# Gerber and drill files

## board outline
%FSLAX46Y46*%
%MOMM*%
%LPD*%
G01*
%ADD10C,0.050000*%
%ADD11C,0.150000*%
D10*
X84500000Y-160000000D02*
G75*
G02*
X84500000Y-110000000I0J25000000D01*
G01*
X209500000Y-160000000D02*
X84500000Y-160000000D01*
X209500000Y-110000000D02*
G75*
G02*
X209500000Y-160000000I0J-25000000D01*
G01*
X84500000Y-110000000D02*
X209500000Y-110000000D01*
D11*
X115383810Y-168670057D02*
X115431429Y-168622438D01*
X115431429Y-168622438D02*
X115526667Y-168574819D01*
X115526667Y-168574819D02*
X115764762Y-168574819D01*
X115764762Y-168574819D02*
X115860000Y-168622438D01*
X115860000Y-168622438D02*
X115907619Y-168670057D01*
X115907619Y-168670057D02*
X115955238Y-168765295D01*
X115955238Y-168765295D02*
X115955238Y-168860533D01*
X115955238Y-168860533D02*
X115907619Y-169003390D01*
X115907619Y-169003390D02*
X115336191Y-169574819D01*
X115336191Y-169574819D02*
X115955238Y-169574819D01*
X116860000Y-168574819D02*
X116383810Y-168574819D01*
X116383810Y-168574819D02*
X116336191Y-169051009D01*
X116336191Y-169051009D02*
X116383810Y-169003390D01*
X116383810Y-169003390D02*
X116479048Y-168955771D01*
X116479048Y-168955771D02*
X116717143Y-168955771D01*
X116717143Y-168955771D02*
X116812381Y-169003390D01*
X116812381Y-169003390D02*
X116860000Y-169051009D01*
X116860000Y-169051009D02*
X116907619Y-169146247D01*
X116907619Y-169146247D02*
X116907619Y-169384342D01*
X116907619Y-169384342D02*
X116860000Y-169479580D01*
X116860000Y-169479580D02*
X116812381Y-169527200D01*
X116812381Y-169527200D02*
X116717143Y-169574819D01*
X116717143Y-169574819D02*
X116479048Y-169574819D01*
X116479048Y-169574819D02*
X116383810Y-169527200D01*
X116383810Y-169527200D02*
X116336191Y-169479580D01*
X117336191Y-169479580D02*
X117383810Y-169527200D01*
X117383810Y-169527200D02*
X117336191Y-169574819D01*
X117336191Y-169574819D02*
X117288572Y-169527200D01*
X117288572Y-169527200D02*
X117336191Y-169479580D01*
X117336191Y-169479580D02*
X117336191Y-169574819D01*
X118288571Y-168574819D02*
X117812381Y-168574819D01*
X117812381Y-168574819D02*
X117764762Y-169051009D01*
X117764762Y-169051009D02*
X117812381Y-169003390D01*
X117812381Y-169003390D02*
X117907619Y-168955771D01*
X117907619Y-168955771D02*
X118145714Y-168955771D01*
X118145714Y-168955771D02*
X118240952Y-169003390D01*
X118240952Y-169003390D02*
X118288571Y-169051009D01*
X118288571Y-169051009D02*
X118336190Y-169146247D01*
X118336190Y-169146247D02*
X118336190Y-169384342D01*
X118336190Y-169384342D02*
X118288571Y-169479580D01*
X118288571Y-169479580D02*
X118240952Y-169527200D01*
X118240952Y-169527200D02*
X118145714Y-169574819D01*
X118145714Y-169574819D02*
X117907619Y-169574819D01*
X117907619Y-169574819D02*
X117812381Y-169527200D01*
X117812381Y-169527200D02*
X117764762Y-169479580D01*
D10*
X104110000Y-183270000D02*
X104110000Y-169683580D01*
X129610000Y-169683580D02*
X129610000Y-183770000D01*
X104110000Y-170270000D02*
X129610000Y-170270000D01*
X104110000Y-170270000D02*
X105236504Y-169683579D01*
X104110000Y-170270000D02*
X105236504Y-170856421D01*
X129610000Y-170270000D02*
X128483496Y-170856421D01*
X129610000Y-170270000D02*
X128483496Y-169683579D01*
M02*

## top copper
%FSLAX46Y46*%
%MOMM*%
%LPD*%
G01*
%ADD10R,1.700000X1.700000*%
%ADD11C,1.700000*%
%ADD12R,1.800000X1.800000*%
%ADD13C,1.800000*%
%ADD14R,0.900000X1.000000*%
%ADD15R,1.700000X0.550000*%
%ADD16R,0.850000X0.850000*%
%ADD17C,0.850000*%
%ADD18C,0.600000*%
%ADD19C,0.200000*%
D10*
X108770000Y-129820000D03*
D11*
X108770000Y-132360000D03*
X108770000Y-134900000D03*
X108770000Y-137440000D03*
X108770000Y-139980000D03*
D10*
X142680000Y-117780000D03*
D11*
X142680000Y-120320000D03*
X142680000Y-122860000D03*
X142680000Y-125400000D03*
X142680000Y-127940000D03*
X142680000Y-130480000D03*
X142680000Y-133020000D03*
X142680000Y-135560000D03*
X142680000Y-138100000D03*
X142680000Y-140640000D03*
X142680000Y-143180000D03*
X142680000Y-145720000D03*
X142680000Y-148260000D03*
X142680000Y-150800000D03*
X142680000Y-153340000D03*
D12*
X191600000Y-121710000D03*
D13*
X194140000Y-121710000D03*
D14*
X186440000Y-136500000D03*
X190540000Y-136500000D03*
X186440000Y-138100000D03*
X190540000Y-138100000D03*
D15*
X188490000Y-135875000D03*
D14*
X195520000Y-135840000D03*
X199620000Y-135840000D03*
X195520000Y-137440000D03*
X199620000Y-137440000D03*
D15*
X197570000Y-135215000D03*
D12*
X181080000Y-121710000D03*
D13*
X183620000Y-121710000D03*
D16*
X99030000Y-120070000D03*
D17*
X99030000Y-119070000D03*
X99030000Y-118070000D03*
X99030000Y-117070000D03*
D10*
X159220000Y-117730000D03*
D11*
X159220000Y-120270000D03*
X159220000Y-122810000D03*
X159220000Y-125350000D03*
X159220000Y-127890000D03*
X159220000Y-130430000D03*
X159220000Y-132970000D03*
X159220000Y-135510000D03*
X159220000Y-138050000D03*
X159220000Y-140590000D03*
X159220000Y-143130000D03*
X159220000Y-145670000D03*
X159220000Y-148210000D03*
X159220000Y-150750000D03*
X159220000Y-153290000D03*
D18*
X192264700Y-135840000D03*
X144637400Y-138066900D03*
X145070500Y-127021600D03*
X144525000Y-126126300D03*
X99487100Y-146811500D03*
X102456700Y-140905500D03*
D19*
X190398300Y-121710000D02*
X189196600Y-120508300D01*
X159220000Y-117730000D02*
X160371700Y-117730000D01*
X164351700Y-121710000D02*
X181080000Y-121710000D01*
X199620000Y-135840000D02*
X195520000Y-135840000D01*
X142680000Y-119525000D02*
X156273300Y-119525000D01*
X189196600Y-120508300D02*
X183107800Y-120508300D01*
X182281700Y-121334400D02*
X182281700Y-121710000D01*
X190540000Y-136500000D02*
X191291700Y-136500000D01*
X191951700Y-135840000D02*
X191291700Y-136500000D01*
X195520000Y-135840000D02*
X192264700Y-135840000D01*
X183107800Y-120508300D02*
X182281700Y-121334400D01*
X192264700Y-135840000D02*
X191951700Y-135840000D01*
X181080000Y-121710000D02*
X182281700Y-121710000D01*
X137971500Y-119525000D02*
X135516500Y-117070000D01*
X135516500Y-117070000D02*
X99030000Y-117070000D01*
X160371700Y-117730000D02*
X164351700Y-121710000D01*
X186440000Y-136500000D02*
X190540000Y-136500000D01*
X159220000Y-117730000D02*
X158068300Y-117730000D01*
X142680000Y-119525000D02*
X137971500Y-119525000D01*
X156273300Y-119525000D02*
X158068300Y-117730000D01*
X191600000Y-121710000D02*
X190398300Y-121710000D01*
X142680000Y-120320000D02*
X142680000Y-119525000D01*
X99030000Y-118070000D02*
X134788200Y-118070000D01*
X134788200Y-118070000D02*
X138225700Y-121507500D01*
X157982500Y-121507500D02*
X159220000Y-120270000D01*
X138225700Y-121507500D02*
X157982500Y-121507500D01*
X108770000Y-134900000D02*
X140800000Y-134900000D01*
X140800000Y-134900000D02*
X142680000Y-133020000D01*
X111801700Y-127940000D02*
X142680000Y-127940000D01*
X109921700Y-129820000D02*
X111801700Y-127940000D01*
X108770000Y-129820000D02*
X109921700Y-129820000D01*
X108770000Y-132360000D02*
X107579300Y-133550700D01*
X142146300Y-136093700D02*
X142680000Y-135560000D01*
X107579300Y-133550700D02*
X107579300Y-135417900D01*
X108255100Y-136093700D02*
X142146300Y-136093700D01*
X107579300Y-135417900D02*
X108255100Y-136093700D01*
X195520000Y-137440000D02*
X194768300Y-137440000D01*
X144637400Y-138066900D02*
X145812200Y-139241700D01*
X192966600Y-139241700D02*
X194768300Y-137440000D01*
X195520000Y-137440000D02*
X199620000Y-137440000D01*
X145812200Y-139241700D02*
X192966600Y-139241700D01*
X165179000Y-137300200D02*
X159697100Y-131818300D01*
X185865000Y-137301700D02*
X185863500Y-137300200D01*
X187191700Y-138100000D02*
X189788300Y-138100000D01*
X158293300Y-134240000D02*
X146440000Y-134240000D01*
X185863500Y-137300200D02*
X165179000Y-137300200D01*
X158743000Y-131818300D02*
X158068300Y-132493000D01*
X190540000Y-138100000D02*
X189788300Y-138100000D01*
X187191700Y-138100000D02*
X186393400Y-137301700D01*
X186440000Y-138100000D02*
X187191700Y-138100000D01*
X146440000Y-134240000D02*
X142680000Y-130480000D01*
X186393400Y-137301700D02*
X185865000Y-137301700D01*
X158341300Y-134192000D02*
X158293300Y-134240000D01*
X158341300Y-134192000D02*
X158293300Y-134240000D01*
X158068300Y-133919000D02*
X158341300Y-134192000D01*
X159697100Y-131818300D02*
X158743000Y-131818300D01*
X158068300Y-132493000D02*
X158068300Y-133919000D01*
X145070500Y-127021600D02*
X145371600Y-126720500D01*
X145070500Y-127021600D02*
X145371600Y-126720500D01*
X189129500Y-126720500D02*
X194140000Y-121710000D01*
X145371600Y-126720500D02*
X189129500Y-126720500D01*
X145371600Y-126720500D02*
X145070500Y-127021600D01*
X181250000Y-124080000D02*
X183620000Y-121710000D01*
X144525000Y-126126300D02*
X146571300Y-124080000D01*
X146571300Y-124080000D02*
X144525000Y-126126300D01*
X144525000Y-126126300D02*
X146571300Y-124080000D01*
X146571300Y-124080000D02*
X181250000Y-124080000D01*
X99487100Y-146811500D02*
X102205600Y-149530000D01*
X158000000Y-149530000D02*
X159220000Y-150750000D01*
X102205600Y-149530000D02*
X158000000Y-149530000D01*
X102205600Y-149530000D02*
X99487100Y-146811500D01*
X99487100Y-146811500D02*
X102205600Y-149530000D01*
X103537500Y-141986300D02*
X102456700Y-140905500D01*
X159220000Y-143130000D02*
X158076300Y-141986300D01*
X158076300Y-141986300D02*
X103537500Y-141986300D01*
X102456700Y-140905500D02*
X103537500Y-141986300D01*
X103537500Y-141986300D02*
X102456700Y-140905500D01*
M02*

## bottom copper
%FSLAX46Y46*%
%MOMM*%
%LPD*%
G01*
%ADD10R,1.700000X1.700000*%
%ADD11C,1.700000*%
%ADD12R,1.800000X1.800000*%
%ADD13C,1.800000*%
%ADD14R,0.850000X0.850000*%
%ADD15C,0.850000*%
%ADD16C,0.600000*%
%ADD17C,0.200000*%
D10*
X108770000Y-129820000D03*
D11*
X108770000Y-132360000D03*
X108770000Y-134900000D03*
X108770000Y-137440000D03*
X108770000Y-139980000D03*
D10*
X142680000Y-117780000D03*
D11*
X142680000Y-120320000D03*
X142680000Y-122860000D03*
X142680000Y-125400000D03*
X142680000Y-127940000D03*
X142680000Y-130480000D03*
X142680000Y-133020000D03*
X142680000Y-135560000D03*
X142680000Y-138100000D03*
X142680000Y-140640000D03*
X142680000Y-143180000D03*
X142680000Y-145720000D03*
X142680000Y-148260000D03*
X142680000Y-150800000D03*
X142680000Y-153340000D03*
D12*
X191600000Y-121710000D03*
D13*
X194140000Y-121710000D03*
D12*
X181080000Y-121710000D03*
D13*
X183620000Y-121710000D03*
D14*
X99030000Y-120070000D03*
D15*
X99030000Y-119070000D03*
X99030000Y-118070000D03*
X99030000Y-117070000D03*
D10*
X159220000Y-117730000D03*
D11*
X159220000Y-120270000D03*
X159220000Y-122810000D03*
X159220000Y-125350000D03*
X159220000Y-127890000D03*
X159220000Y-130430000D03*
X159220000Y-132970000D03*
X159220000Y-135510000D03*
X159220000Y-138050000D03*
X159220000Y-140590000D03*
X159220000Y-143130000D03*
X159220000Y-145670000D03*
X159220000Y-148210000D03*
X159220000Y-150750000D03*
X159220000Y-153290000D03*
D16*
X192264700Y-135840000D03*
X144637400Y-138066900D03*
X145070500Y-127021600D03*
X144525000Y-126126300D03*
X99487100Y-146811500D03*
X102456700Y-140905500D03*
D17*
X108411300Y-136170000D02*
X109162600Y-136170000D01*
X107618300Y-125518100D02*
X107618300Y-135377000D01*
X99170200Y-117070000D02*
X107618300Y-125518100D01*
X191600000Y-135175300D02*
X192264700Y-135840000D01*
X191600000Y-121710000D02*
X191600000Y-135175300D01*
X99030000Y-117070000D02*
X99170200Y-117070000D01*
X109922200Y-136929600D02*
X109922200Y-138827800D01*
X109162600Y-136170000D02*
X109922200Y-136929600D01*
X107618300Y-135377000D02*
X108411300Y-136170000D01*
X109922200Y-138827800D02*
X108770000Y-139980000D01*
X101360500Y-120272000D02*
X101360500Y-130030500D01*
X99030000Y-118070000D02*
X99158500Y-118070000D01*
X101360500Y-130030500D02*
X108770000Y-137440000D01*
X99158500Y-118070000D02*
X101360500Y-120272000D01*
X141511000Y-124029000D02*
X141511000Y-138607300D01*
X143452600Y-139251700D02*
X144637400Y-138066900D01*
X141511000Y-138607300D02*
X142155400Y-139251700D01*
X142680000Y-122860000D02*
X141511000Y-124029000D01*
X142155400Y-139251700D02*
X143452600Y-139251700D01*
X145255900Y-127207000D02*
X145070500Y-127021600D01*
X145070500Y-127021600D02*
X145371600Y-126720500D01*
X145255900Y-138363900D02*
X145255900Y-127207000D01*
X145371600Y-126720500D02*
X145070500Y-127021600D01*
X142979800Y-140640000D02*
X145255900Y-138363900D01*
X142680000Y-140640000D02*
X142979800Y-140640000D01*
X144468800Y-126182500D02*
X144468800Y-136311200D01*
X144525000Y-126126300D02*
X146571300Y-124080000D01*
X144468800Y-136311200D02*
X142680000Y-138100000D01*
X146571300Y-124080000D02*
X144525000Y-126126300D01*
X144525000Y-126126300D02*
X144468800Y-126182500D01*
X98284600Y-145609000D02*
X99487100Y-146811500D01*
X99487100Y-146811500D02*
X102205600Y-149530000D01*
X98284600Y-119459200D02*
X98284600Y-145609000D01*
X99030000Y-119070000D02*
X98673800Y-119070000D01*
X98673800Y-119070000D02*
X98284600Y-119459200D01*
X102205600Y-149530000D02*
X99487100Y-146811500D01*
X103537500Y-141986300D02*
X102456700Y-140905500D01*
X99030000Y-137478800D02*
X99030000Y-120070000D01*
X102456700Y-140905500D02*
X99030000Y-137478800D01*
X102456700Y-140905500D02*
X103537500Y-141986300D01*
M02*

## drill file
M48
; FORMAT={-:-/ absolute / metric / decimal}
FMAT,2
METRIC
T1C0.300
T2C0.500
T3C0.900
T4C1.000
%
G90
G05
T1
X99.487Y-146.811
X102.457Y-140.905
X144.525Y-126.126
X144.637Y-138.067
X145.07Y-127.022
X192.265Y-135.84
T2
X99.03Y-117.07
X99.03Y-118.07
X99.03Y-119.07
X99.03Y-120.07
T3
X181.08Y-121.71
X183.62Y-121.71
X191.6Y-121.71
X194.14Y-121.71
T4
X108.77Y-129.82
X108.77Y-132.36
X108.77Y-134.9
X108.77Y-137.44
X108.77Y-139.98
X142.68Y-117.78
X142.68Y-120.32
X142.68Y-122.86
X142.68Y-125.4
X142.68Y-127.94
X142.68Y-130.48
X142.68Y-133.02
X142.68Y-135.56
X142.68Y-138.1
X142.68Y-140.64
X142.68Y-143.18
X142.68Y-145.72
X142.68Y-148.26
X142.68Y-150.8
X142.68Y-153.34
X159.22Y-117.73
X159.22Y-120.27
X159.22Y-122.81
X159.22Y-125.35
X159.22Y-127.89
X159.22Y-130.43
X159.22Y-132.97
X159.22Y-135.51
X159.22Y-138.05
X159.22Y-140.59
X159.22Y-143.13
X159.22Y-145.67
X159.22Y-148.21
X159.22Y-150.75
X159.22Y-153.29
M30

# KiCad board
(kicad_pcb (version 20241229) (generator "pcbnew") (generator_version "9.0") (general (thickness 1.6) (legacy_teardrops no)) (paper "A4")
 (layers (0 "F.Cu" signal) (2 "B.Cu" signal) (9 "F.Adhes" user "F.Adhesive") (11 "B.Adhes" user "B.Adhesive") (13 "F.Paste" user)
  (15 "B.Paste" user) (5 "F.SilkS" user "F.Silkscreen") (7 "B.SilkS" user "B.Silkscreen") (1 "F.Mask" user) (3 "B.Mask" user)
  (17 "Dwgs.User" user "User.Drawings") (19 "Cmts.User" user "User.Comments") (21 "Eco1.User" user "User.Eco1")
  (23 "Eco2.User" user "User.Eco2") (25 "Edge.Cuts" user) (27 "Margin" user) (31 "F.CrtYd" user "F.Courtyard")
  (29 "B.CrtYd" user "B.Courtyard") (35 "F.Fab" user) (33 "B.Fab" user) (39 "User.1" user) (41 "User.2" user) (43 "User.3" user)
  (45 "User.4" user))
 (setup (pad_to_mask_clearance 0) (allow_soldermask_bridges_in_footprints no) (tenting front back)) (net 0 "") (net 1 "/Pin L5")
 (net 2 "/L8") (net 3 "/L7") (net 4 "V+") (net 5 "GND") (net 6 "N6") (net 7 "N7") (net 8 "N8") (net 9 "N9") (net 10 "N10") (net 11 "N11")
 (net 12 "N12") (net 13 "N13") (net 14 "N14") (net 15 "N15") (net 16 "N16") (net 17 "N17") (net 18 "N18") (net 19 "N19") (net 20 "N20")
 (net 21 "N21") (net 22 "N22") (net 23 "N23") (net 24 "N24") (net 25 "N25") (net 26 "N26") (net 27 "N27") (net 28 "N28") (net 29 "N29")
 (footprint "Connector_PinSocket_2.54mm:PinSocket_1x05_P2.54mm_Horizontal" (layer "F.Cu") (at 108.77 129.82)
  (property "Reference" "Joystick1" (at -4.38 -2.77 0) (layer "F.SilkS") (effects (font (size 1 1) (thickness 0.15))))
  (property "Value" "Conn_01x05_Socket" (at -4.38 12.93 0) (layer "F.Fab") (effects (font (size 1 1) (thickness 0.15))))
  (pad "1" thru_hole rect (at 0 0) (size 1.7 1.7) (drill 1) (layers "*.Cu" "*.Mask") (remove_unused_layers no) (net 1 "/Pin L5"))
  (pad "2" thru_hole circle (at 0 2.54) (size 1.7 1.7) (drill 1) (layers "*.Cu" "*.Mask") (remove_unused_layers no) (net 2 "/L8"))
  (pad "3" thru_hole circle (at 0 5.08) (size 1.7 1.7) (drill 1) (layers "*.Cu" "*.Mask") (remove_unused_layers no) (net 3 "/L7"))
  (pad "4" thru_hole circle (at 0 7.62) (size 1.7 1.7) (drill 1) (layers "*.Cu" "*.Mask") (remove_unused_layers no) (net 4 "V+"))
  (pad "5" thru_hole circle (at 0 10.16) (size 1.7 1.7) (drill 1) (layers "*.Cu" "*.Mask") (remove_unused_layers no) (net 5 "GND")))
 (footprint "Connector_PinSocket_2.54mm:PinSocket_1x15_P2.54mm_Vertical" (layer "F.Cu") (at 142.68 117.78)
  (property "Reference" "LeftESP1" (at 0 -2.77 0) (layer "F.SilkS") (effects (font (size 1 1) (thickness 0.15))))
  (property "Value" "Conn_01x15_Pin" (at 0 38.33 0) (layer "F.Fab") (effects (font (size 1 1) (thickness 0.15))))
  (pad "1" thru_hole rect (at 0 0) (size 1.7 1.7) (drill 1) (layers "*.Cu" "*.Mask") (remove_unused_layers no) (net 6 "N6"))
  (pad "2" thru_hole circle (at 0 2.54) (size 1.7 1.7) (drill 1) (layers "*.Cu" "*.Mask") (remove_unused_layers no) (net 5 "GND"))
  (pad "3" thru_hole circle (at 0 5.08) (size 1.7 1.7) (drill 1) (layers "*.Cu" "*.Mask") (remove_unused_layers no) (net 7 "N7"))
  (pad "4" thru_hole circle (at 0 7.62) (size 1.7 1.7) (drill 1) (layers "*.Cu" "*.Mask") (remove_unused_layers no) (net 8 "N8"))
  (pad "5" thru_hole circle (at 0 10.16) (size 1.7 1.7) (drill 1) (layers "*.Cu" "*.Mask") (remove_unused_layers no) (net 1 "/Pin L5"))
  (pad "6" thru_hole circle (at 0 12.7) (size 1.7 1.7) (drill 1) (layers "*.Cu" "*.Mask") (remove_unused_layers no) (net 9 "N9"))
  (pad "7" thru_hole circle (at 0 15.24) (size 1.7 1.7) (drill 1) (layers "*.Cu" "*.Mask") (remove_unused_layers no) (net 3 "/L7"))
  (pad "8" thru_hole circle (at 0 17.78) (size 1.7 1.7) (drill 1) (layers "*.Cu" "*.Mask") (remove_unused_layers no) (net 2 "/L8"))
  (pad "9" thru_hole circle (at 0 20.32) (size 1.7 1.7) (drill 1) (layers "*.Cu" "*.Mask") (remove_unused_layers no) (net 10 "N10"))
  (pad "10" thru_hole circle (at 0 22.86) (size 1.7 1.7) (drill 1) (layers "*.Cu" "*.Mask") (remove_unused_layers no) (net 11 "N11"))
  (pad "11" thru_hole circle (at 0 25.4) (size 1.7 1.7) (drill 1) (layers "*.Cu" "*.Mask") (remove_unused_layers no) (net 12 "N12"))
  (pad "12" thru_hole circle (at 0 27.94) (size 1.7 1.7) (drill 1) (layers "*.Cu" "*.Mask") (remove_unused_layers no) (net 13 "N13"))
  (pad "13" thru_hole circle (at 0 30.48) (size 1.7 1.7) (drill 1) (layers "*.Cu" "*.Mask") (remove_unused_layers no) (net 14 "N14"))
  (pad "14" thru_hole circle (at 0 33.02) (size 1.7 1.7) (drill 1) (layers "*.Cu" "*.Mask") (remove_unused_layers no) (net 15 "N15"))
  (pad "15" thru_hole circle (at 0 35.56) (size 1.7 1.7) (drill 1) (layers "*.Cu" "*.Mask") (remove_unused_layers no) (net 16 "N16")))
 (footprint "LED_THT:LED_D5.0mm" (layer "F.Cu") (at 191.6 121.71)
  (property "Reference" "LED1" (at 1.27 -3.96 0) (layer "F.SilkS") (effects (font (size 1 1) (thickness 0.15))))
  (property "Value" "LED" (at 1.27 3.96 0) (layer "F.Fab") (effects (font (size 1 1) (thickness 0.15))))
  (pad "1" thru_hole rect (at 0 0) (size 1.8 1.8) (drill 0.9) (layers "*.Cu" "*.Mask") (remove_unused_layers no) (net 5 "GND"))
  (pad "2" thru_hole circle (at 2.54 0) (size 1.8 1.8) (drill 0.9) (layers "*.Cu" "*.Mask") (remove_unused_layers no) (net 11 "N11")))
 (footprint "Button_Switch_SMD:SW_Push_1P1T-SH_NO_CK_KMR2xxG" (layer "F.Cu") (at 188.49 137.3)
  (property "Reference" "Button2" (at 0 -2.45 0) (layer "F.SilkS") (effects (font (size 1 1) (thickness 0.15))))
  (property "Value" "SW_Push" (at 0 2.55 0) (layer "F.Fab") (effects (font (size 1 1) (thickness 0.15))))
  (pad "1" smd rect (at -2.05 -0.8) (size 0.9 1) (layers "F.Cu" "F.Mask" "F.Paste") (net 5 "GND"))
  (pad "1" smd rect (at 2.05 -0.8) (size 0.9 1) (layers "F.Cu" "F.Mask" "F.Paste") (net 5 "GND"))
  (pad "2" smd rect (at -2.05 0.8) (size 0.9 1) (layers "F.Cu" "F.Mask" "F.Paste") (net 9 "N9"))
  (pad "2" smd rect (at 2.05 0.8) (size 0.9 1) (layers "F.Cu" "F.Mask" "F.Paste") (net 9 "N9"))
  (pad "SH" smd rect (at 0 -1.425) (size 1.7 0.55) (layers "F.Cu" "F.Mask" "F.Paste")))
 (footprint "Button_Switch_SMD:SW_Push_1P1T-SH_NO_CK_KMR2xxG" (layer "F.Cu") (at 197.57 136.64)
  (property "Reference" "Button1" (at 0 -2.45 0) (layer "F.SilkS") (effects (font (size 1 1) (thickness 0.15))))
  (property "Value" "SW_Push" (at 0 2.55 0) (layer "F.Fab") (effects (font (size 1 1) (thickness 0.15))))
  (pad "1" smd rect (at -2.05 -0.8) (size 0.9 1) (layers "F.Cu" "F.Mask" "F.Paste") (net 5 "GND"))
  (pad "1" smd rect (at 2.05 -0.8) (size 0.9 1) (layers "F.Cu" "F.Mask" "F.Paste") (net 5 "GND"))
  (pad "2" smd rect (at -2.05 0.8) (size 0.9 1) (layers "F.Cu" "F.Mask" "F.Paste") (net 7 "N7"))
  (pad "2" smd rect (at 2.05 0.8) (size 0.9 1) (layers "F.Cu" "F.Mask" "F.Paste") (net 7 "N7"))
  (pad "SH" smd rect (at 0 -1.425) (size 1.7 0.55) (layers "F.Cu" "F.Mask" "F.Paste")))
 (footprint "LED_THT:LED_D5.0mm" (layer "F.Cu") (at 181.08 121.71)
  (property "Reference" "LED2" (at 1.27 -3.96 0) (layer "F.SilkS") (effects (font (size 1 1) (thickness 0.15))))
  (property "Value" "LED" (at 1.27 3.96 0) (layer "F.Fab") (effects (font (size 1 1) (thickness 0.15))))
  (pad "1" thru_hole rect (at 0 0) (size 1.8 1.8) (drill 0.9) (layers "*.Cu" "*.Mask") (remove_unused_layers no) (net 5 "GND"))
  (pad "2" thru_hole circle (at 2.54 0) (size 1.8 1.8) (drill 0.9) (layers "*.Cu" "*.Mask") (remove_unused_layers no) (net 10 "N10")))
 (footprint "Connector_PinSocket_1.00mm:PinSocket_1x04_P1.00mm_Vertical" (layer "F.Cu") (at 99.03 120.07 180)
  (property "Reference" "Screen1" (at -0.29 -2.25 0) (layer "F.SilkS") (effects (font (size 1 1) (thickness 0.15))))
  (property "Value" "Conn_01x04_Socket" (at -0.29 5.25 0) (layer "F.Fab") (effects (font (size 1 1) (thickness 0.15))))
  (pad "1" thru_hole rect (at 0 0 180) (size 0.85 0.85) (drill 0.5) (layers "*.Cu" "*.Mask") (remove_unused_layers no) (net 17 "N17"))
  (pad "2" thru_hole circle (at 0 1 180) (size 0.85 0.85) (drill 0.5) (layers "*.Cu" "*.Mask") (remove_unused_layers no) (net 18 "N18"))
  (pad "3" thru_hole circle (at 0 2 180) (size 0.85 0.85) (drill 0.5) (layers "*.Cu" "*.Mask") (remove_unused_layers no) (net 4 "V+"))
  (pad "4" thru_hole circle (at 0 3 180) (size 0.85 0.85) (drill 0.5) (layers "*.Cu" "*.Mask") (remove_unused_layers no) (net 5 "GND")))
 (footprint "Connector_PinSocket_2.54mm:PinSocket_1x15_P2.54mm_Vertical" (layer "F.Cu") (at 159.22 117.73)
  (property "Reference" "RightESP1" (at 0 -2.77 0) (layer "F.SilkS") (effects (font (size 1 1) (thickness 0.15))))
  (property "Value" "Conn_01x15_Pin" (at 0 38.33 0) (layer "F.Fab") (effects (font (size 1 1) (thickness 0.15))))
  (pad "1" thru_hole rect (at 0 0) (size 1.7 1.7) (drill 1) (layers "*.Cu" "*.Mask") (remove_unused_layers no) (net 5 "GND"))
  (pad "2" thru_hole circle (at 0 2.54) (size 1.7 1.7) (drill 1) (layers "*.Cu" "*.Mask") (remove_unused_layers no) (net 4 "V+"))
  (pad "3" thru_hole circle (at 0 5.08) (size 1.7 1.7) (drill 1) (layers "*.Cu" "*.Mask") (remove_unused_layers no) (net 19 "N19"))
  (pad "4" thru_hole circle (at 0 7.62) (size 1.7 1.7) (drill 1) (layers "*.Cu" "*.Mask") (remove_unused_layers no) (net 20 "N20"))
  (pad "5" thru_hole circle (at 0 10.16) (size 1.7 1.7) (drill 1) (layers "*.Cu" "*.Mask") (remove_unused_layers no) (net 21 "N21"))
  (pad "6" thru_hole circle (at 0 12.7) (size 1.7 1.7) (drill 1) (layers "*.Cu" "*.Mask") (remove_unused_layers no) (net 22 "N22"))
  (pad "7" thru_hole circle (at 0 15.24) (size 1.7 1.7) (drill 1) (layers "*.Cu" "*.Mask") (remove_unused_layers no) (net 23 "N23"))
  (pad "8" thru_hole circle (at 0 17.78) (size 1.7 1.7) (drill 1) (layers "*.Cu" "*.Mask") (remove_unused_layers no) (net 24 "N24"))
  (pad "9" thru_hole circle (at 0 20.32) (size 1.7 1.7) (drill 1) (layers "*.Cu" "*.Mask") (remove_unused_layers no) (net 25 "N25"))
  (pad "10" thru_hole circle (at 0 22.86) (size 1.7 1.7) (drill 1) (layers "*.Cu" "*.Mask") (remove_unused_layers no) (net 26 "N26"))
  (pad "11" thru_hole circle (at 0 25.4) (size 1.7 1.7) (drill 1) (layers "*.Cu" "*.Mask") (remove_unused_layers no) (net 17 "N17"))
  (pad "12" thru_hole circle (at 0 27.94) (size 1.7 1.7) (drill 1) (layers "*.Cu" "*.Mask") (remove_unused_layers no) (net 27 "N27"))
  (pad "13" thru_hole circle (at 0 30.48) (size 1.7 1.7) (drill 1) (layers "*.Cu" "*.Mask") (remove_unused_layers no) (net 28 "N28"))
  (pad "14" thru_hole circle (at 0 33.02) (size 1.7 1.7) (drill 1) (layers "*.Cu" "*.Mask") (remove_unused_layers no) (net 18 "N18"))
  (pad "15" thru_hole circle (at 0 35.56) (size 1.7 1.7) (drill 1) (layers "*.Cu" "*.Mask") (remove_unused_layers no) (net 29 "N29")))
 (gr_arc (start 84.5 160) (mid 59.5 135) (end 84.5 110) (stroke (width 0.05) (type default)) (layer "Edge.Cuts"))
 (gr_line (start 209.5 160) (end 84.5 160) (stroke (width 0.05) (type default)) (layer "Edge.Cuts"))
 (gr_arc (start 209.5 110) (mid 234.5 135) (end 209.5 160) (stroke (width 0.05) (type default)) (layer "Edge.Cuts"))
 (gr_line (start 84.5 110) (end 209.5 110) (stroke (width 0.05) (type default)) (layer "Edge.Cuts"))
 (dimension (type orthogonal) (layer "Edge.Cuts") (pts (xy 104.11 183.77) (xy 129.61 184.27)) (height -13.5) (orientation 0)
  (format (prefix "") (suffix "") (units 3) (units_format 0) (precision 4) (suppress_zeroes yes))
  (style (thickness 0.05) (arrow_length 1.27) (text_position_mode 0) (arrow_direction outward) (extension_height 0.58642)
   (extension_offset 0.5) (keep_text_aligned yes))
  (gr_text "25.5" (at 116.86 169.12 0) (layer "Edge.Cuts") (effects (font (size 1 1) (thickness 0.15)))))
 (segment (start 190.3983 121.71) (end 189.1966 120.5083) (width 0.2) (layer "F.Cu") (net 5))
 (segment (start 159.22 117.73) (end 160.3717 117.73) (width 0.2) (layer "F.Cu") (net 5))
 (segment (start 164.3517 121.71) (end 181.08 121.71) (width 0.2) (layer "F.Cu") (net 5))
 (segment (start 199.62 135.84) (end 195.52 135.84) (width 0.2) (layer "F.Cu") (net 5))
 (segment (start 142.68 119.525) (end 156.2733 119.525) (width 0.2) (layer "F.Cu") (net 5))
 (segment (start 189.1966 120.5083) (end 183.1078 120.5083) (width 0.2) (layer "F.Cu") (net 5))
 (segment (start 182.2817 121.3344) (end 182.2817 121.71) (width 0.2) (layer "F.Cu") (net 5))
 (segment (start 190.54 136.5) (end 191.2917 136.5) (width 0.2) (layer "F.Cu") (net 5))
 (segment (start 191.9517 135.84) (end 191.2917 136.5) (width 0.2) (layer "F.Cu") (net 5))
 (segment (start 195.52 135.84) (end 192.2647 135.84) (width 0.2) (layer "F.Cu") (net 5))
 (segment (start 183.1078 120.5083) (end 182.2817 121.3344) (width 0.2) (layer "F.Cu") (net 5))
 (segment (start 192.2647 135.84) (end 191.9517 135.84) (width 0.2) (layer "F.Cu") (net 5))
 (segment (start 181.08 121.71) (end 182.2817 121.71) (width 0.2) (layer "F.Cu") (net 5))
 (segment (start 137.9715 119.525) (end 135.5165 117.07) (width 0.2) (layer "F.Cu") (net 5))
 (segment (start 135.5165 117.07) (end 99.03 117.07) (width 0.2) (layer "F.Cu") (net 5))
 (segment (start 160.3717 117.73) (end 164.3517 121.71) (width 0.2) (layer "F.Cu") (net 5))
 (segment (start 186.44 136.5) (end 190.54 136.5) (width 0.2) (layer "F.Cu") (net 5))
 (segment (start 159.22 117.73) (end 158.0683 117.73) (width 0.2) (layer "F.Cu") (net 5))
 (segment (start 142.68 119.525) (end 137.9715 119.525) (width 0.2) (layer "F.Cu") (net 5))
 (segment (start 156.2733 119.525) (end 158.0683 117.73) (width 0.2) (layer "F.Cu") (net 5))
 (segment (start 191.6 121.71) (end 190.3983 121.71) (width 0.2) (layer "F.Cu") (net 5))
 (segment (start 142.68 120.32) (end 142.68 119.525) (width 0.2) (layer "F.Cu") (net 5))
 (via (at 192.2647 135.84) (size 0.6) (drill 0.3) (layers "F.Cu" "B.Cu") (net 5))
 (segment (start 108.4113 136.17) (end 109.1626 136.17) (width 0.2) (layer "B.Cu") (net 5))
 (segment (start 107.6183 125.5181) (end 107.6183 135.377) (width 0.2) (layer "B.Cu") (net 5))
 (segment (start 99.1702 117.07) (end 107.6183 125.5181) (width 0.2) (layer "B.Cu") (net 5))
 (segment (start 191.6 135.1753) (end 192.2647 135.84) (width 0.2) (layer "B.Cu") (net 5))
 (segment (start 191.6 121.71) (end 191.6 135.1753) (width 0.2) (layer "B.Cu") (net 5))
 (segment (start 99.03 117.07) (end 99.1702 117.07) (width 0.2) (layer "B.Cu") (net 5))
 (segment (start 109.9222 136.9296) (end 109.9222 138.8278) (width 0.2) (layer "B.Cu") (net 5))
 (segment (start 109.1626 136.17) (end 109.9222 136.9296) (width 0.2) (layer "B.Cu") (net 5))
 (segment (start 107.6183 135.377) (end 108.4113 136.17) (width 0.2) (layer "B.Cu") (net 5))
 (segment (start 109.9222 138.8278) (end 108.77 139.98) (width 0.2) (layer "B.Cu") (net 5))
 (segment (start 99.03 118.07) (end 134.7882 118.07) (width 0.2) (layer "F.Cu") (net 4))
 (segment (start 134.7882 118.07) (end 138.2257 121.5075) (width 0.2) (layer "F.Cu") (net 4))
 (segment (start 157.9825 121.5075) (end 159.22 120.27) (width 0.2) (layer "F.Cu") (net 4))
 (segment (start 138.2257 121.5075) (end 157.9825 121.5075) (width 0.2) (layer "F.Cu") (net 4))
 (segment (start 101.3605 120.272) (end 101.3605 130.0305) (width 0.2) (layer "B.Cu") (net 4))
 (segment (start 99.03 118.07) (end 99.1585 118.07) (width 0.2) (layer "B.Cu") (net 4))
 (segment (start 101.3605 130.0305) (end 108.77 137.44) (width 0.2) (layer "B.Cu") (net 4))
 (segment (start 99.1585 118.07) (end 101.3605 120.272) (width 0.2) (layer "B.Cu") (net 4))
 (segment (start 108.77 134.9) (end 140.8 134.9) (width 0.2) (layer "F.Cu") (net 3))
 (segment (start 140.8 134.9) (end 142.68 133.02) (width 0.2) (layer "F.Cu") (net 3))
 (segment (start 111.8017 127.94) (end 142.68 127.94) (width 0.2) (layer "F.Cu") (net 1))
 (segment (start 109.9217 129.82) (end 111.8017 127.94) (width 0.2) (layer "F.Cu") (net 1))
 (segment (start 108.77 129.82) (end 109.9217 129.82) (width 0.2) (layer "F.Cu") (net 1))
 (segment (start 108.77 132.36) (end 107.5793 133.5507) (width 0.2) (layer "F.Cu") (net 2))
 (segment (start 142.1463 136.0937) (end 142.68 135.56) (width 0.2) (layer "F.Cu") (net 2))
 (segment (start 107.5793 133.5507) (end 107.5793 135.4179) (width 0.2) (layer "F.Cu") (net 2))
 (segment (start 108.2551 136.0937) (end 142.1463 136.0937) (width 0.2) (layer "F.Cu") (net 2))
 (segment (start 107.5793 135.4179) (end 108.2551 136.0937) (width 0.2) (layer "F.Cu") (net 2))
 (segment (start 195.52 137.44) (end 194.7683 137.44) (width 0.2) (layer "F.Cu") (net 7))
 (segment (start 144.6374 138.0669) (end 145.8122 139.2417) (width 0.2) (layer "F.Cu") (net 7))
 (segment (start 192.9666 139.2417) (end 194.7683 137.44) (width 0.2) (layer "F.Cu") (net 7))
 (segment (start 195.52 137.44) (end 199.62 137.44) (width 0.2) (layer "F.Cu") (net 7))
 (segment (start 145.8122 139.2417) (end 192.9666 139.2417) (width 0.2) (layer "F.Cu") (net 7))
 (via (at 144.6374 138.0669) (size 0.6) (drill 0.3) (layers "F.Cu" "B.Cu") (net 7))
 (segment (start 141.511 124.029) (end 141.511 138.6073) (width 0.2) (layer "B.Cu") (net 7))
 (segment (start 143.4526 139.2517) (end 144.6374 138.0669) (width 0.2) (layer "B.Cu") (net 7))
 (segment (start 141.511 138.6073) (end 142.1554 139.2517) (width 0.2) (layer "B.Cu") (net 7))
 (segment (start 142.68 122.86) (end 141.511 124.029) (width 0.2) (layer "B.Cu") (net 7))
 (segment (start 142.1554 139.2517) (end 143.4526 139.2517) (width 0.2) (layer "B.Cu") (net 7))
 (segment (start 165.179 137.3002) (end 159.6971 131.8183) (width 0.2) (layer "F.Cu") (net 9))
 (segment (start 185.865 137.3017) (end 185.8635 137.3002) (width 0.2) (layer "F.Cu") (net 9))
 (segment (start 187.1917 138.1) (end 189.7883 138.1) (width 0.2) (layer "F.Cu") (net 9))
 (segment (start 158.2933 134.24) (end 146.44 134.24) (width 0.2) (layer "F.Cu") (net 9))
 (segment (start 185.8635 137.3002) (end 165.179 137.3002) (width 0.2) (layer "F.Cu") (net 9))
 (segment (start 158.743 131.8183) (end 158.0683 132.493) (width 0.2) (layer "F.Cu") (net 9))
 (segment (start 190.54 138.1) (end 189.7883 138.1) (width 0.2) (layer "F.Cu") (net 9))
 (segment (start 187.1917 138.1) (end 186.3934 137.3017) (width 0.2) (layer "F.Cu") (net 9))
 (segment (start 186.44 138.1) (end 187.1917 138.1) (width 0.2) (layer "F.Cu") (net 9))
 (segment (start 146.44 134.24) (end 142.68 130.48) (width 0.2) (layer "F.Cu") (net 9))
 (segment (start 186.3934 137.3017) (end 185.865 137.3017) (width 0.2) (layer "F.Cu") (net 9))
 (segment (start 158.3413 134.192) (end 158.2933 134.24) (width 0.2) (layer "F.Cu") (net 9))
 (segment (start 158.3413 134.192) (end 158.2933 134.24) (width 0.2) (layer "F.Cu") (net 9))
 (segment (start 158.0683 133.919) (end 158.3413 134.192) (width 0.2) (layer "F.Cu") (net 9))
 (segment (start 159.6971 131.8183) (end 158.743 131.8183) (width 0.2) (layer "F.Cu") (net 9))
 (segment (start 158.0683 132.493) (end 158.0683 133.919) (width 0.2) (layer "F.Cu") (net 9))
 (segment (start 145.0705 127.0216) (end 145.3716 126.7205) (width 0.2) (layer "F.Cu") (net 11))
 (segment (start 145.0705 127.0216) (end 145.3716 126.7205) (width 0.2) (layer "F.Cu") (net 11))
 (segment (start 189.1295 126.7205) (end 194.14 121.71) (width 0.2) (layer "F.Cu") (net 11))
 (segment (start 145.3716 126.7205) (end 189.1295 126.7205) (width 0.2) (layer "F.Cu") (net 11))
 (segment (start 145.3716 126.7205) (end 145.0705 127.0216) (width 0.2) (layer "F.Cu") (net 11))
 (via (at 145.0705 127.0216) (size 0.6) (drill 0.3) (layers "F.Cu" "B.Cu") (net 11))
 (segment (start 145.2559 127.207) (end 145.0705 127.0216) (width 0.2) (layer "B.Cu") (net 11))
 (segment (start 145.0705 127.0216) (end 145.3716 126.7205) (width 0.2) (layer "B.Cu") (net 11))
 (segment (start 145.2559 138.3639) (end 145.2559 127.207) (width 0.2) (layer "B.Cu") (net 11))
 (segment (start 145.3716 126.7205) (end 145.0705 127.0216) (width 0.2) (layer "B.Cu") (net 11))
 (segment (start 142.9798 140.64) (end 145.2559 138.3639) (width 0.2) (layer "B.Cu") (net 11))
 (segment (start 142.68 140.64) (end 142.9798 140.64) (width 0.2) (layer "B.Cu") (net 11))
 (segment (start 181.25 124.08) (end 183.62 121.71) (width 0.2) (layer "F.Cu") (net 10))
 (segment (start 144.525 126.1263) (end 146.5713 124.08) (width 0.2) (layer "F.Cu") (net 10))
 (segment (start 146.5713 124.08) (end 144.525 126.1263) (width 0.2) (layer "F.Cu") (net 10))
 (segment (start 144.525 126.1263) (end 146.5713 124.08) (width 0.2) (layer "F.Cu") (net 10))
 (segment (start 146.5713 124.08) (end 181.25 124.08) (width 0.2) (layer "F.Cu") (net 10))
 (via (at 144.525 126.1263) (size 0.6) (drill 0.3) (layers "F.Cu" "B.Cu") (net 10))
 (segment (start 144.4688 126.1825) (end 144.4688 136.3112) (width 0.2) (layer "B.Cu") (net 10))
 (segment (start 144.525 126.1263) (end 146.5713 124.08) (width 0.2) (layer "B.Cu") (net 10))
 (segment (start 144.4688 136.3112) (end 142.68 138.1) (width 0.2) (layer "B.Cu") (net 10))
 (segment (start 146.5713 124.08) (end 144.525 126.1263) (width 0.2) (layer "B.Cu") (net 10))
 (segment (start 144.525 126.1263) (end 144.4688 126.1825) (width 0.2) (layer "B.Cu") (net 10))
 (segment (start 99.4871 146.8115) (end 102.2056 149.53) (width 0.2) (layer "F.Cu") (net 18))
 (segment (start 158 149.53) (end 159.22 150.75) (width 0.2) (layer "F.Cu") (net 18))
 (segment (start 102.2056 149.53) (end 158 149.53) (width 0.2) (layer "F.Cu") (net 18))
 (segment (start 102.2056 149.53) (end 99.4871 146.8115) (width 0.2) (layer "F.Cu") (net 18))
 (segment (start 99.4871 146.8115) (end 102.2056 149.53) (width 0.2) (layer "F.Cu") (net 18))
 (via (at 99.4871 146.8115) (size 0.6) (drill 0.3) (layers "F.Cu" "B.Cu") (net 18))
 (segment (start 98.2846 145.609) (end 99.4871 146.8115) (width 0.2) (layer "B.Cu") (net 18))
 (segment (start 99.4871 146.8115) (end 102.2056 149.53) (width 0.2) (layer "B.Cu") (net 18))
 (segment (start 98.2846 119.4592) (end 98.2846 145.609) (width 0.2) (layer "B.Cu") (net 18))
 (segment (start 99.03 119.07) (end 98.6738 119.07) (width 0.2) (layer "B.Cu") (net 18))
 (segment (start 98.6738 119.07) (end 98.2846 119.4592) (width 0.2) (layer "B.Cu") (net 18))
 (segment (start 102.2056 149.53) (end 99.4871 146.8115) (width 0.2) (layer "B.Cu") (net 18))
 (segment (start 103.5375 141.9863) (end 102.4567 140.9055) (width 0.2) (layer "F.Cu") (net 17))
 (segment (start 159.22 143.13) (end 158.0763 141.9863) (width 0.2) (layer "F.Cu") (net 17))
 (segment (start 158.0763 141.9863) (end 103.5375 141.9863) (width 0.2) (layer "F.Cu") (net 17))
 (segment (start 102.4567 140.9055) (end 103.5375 141.9863) (width 0.2) (layer "F.Cu") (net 17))
 (segment (start 103.5375 141.9863) (end 102.4567 140.9055) (width 0.2) (layer "F.Cu") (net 17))
 (via (at 102.4567 140.9055) (size 0.6) (drill 0.3) (layers "F.Cu" "B.Cu") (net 17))
 (segment (start 103.5375 141.9863) (end 102.4567 140.9055) (width 0.2) (layer "B.Cu") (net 17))
 (segment (start 99.03 137.4788) (end 99.03 120.07) (width 0.2) (layer "B.Cu") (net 17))
 (segment (start 102.4567 140.9055) (end 99.03 137.4788) (width 0.2) (layer "B.Cu") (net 17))
 (segment (start 102.4567 140.9055) (end 103.5375 141.9863) (width 0.2) (layer "B.Cu") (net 17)))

